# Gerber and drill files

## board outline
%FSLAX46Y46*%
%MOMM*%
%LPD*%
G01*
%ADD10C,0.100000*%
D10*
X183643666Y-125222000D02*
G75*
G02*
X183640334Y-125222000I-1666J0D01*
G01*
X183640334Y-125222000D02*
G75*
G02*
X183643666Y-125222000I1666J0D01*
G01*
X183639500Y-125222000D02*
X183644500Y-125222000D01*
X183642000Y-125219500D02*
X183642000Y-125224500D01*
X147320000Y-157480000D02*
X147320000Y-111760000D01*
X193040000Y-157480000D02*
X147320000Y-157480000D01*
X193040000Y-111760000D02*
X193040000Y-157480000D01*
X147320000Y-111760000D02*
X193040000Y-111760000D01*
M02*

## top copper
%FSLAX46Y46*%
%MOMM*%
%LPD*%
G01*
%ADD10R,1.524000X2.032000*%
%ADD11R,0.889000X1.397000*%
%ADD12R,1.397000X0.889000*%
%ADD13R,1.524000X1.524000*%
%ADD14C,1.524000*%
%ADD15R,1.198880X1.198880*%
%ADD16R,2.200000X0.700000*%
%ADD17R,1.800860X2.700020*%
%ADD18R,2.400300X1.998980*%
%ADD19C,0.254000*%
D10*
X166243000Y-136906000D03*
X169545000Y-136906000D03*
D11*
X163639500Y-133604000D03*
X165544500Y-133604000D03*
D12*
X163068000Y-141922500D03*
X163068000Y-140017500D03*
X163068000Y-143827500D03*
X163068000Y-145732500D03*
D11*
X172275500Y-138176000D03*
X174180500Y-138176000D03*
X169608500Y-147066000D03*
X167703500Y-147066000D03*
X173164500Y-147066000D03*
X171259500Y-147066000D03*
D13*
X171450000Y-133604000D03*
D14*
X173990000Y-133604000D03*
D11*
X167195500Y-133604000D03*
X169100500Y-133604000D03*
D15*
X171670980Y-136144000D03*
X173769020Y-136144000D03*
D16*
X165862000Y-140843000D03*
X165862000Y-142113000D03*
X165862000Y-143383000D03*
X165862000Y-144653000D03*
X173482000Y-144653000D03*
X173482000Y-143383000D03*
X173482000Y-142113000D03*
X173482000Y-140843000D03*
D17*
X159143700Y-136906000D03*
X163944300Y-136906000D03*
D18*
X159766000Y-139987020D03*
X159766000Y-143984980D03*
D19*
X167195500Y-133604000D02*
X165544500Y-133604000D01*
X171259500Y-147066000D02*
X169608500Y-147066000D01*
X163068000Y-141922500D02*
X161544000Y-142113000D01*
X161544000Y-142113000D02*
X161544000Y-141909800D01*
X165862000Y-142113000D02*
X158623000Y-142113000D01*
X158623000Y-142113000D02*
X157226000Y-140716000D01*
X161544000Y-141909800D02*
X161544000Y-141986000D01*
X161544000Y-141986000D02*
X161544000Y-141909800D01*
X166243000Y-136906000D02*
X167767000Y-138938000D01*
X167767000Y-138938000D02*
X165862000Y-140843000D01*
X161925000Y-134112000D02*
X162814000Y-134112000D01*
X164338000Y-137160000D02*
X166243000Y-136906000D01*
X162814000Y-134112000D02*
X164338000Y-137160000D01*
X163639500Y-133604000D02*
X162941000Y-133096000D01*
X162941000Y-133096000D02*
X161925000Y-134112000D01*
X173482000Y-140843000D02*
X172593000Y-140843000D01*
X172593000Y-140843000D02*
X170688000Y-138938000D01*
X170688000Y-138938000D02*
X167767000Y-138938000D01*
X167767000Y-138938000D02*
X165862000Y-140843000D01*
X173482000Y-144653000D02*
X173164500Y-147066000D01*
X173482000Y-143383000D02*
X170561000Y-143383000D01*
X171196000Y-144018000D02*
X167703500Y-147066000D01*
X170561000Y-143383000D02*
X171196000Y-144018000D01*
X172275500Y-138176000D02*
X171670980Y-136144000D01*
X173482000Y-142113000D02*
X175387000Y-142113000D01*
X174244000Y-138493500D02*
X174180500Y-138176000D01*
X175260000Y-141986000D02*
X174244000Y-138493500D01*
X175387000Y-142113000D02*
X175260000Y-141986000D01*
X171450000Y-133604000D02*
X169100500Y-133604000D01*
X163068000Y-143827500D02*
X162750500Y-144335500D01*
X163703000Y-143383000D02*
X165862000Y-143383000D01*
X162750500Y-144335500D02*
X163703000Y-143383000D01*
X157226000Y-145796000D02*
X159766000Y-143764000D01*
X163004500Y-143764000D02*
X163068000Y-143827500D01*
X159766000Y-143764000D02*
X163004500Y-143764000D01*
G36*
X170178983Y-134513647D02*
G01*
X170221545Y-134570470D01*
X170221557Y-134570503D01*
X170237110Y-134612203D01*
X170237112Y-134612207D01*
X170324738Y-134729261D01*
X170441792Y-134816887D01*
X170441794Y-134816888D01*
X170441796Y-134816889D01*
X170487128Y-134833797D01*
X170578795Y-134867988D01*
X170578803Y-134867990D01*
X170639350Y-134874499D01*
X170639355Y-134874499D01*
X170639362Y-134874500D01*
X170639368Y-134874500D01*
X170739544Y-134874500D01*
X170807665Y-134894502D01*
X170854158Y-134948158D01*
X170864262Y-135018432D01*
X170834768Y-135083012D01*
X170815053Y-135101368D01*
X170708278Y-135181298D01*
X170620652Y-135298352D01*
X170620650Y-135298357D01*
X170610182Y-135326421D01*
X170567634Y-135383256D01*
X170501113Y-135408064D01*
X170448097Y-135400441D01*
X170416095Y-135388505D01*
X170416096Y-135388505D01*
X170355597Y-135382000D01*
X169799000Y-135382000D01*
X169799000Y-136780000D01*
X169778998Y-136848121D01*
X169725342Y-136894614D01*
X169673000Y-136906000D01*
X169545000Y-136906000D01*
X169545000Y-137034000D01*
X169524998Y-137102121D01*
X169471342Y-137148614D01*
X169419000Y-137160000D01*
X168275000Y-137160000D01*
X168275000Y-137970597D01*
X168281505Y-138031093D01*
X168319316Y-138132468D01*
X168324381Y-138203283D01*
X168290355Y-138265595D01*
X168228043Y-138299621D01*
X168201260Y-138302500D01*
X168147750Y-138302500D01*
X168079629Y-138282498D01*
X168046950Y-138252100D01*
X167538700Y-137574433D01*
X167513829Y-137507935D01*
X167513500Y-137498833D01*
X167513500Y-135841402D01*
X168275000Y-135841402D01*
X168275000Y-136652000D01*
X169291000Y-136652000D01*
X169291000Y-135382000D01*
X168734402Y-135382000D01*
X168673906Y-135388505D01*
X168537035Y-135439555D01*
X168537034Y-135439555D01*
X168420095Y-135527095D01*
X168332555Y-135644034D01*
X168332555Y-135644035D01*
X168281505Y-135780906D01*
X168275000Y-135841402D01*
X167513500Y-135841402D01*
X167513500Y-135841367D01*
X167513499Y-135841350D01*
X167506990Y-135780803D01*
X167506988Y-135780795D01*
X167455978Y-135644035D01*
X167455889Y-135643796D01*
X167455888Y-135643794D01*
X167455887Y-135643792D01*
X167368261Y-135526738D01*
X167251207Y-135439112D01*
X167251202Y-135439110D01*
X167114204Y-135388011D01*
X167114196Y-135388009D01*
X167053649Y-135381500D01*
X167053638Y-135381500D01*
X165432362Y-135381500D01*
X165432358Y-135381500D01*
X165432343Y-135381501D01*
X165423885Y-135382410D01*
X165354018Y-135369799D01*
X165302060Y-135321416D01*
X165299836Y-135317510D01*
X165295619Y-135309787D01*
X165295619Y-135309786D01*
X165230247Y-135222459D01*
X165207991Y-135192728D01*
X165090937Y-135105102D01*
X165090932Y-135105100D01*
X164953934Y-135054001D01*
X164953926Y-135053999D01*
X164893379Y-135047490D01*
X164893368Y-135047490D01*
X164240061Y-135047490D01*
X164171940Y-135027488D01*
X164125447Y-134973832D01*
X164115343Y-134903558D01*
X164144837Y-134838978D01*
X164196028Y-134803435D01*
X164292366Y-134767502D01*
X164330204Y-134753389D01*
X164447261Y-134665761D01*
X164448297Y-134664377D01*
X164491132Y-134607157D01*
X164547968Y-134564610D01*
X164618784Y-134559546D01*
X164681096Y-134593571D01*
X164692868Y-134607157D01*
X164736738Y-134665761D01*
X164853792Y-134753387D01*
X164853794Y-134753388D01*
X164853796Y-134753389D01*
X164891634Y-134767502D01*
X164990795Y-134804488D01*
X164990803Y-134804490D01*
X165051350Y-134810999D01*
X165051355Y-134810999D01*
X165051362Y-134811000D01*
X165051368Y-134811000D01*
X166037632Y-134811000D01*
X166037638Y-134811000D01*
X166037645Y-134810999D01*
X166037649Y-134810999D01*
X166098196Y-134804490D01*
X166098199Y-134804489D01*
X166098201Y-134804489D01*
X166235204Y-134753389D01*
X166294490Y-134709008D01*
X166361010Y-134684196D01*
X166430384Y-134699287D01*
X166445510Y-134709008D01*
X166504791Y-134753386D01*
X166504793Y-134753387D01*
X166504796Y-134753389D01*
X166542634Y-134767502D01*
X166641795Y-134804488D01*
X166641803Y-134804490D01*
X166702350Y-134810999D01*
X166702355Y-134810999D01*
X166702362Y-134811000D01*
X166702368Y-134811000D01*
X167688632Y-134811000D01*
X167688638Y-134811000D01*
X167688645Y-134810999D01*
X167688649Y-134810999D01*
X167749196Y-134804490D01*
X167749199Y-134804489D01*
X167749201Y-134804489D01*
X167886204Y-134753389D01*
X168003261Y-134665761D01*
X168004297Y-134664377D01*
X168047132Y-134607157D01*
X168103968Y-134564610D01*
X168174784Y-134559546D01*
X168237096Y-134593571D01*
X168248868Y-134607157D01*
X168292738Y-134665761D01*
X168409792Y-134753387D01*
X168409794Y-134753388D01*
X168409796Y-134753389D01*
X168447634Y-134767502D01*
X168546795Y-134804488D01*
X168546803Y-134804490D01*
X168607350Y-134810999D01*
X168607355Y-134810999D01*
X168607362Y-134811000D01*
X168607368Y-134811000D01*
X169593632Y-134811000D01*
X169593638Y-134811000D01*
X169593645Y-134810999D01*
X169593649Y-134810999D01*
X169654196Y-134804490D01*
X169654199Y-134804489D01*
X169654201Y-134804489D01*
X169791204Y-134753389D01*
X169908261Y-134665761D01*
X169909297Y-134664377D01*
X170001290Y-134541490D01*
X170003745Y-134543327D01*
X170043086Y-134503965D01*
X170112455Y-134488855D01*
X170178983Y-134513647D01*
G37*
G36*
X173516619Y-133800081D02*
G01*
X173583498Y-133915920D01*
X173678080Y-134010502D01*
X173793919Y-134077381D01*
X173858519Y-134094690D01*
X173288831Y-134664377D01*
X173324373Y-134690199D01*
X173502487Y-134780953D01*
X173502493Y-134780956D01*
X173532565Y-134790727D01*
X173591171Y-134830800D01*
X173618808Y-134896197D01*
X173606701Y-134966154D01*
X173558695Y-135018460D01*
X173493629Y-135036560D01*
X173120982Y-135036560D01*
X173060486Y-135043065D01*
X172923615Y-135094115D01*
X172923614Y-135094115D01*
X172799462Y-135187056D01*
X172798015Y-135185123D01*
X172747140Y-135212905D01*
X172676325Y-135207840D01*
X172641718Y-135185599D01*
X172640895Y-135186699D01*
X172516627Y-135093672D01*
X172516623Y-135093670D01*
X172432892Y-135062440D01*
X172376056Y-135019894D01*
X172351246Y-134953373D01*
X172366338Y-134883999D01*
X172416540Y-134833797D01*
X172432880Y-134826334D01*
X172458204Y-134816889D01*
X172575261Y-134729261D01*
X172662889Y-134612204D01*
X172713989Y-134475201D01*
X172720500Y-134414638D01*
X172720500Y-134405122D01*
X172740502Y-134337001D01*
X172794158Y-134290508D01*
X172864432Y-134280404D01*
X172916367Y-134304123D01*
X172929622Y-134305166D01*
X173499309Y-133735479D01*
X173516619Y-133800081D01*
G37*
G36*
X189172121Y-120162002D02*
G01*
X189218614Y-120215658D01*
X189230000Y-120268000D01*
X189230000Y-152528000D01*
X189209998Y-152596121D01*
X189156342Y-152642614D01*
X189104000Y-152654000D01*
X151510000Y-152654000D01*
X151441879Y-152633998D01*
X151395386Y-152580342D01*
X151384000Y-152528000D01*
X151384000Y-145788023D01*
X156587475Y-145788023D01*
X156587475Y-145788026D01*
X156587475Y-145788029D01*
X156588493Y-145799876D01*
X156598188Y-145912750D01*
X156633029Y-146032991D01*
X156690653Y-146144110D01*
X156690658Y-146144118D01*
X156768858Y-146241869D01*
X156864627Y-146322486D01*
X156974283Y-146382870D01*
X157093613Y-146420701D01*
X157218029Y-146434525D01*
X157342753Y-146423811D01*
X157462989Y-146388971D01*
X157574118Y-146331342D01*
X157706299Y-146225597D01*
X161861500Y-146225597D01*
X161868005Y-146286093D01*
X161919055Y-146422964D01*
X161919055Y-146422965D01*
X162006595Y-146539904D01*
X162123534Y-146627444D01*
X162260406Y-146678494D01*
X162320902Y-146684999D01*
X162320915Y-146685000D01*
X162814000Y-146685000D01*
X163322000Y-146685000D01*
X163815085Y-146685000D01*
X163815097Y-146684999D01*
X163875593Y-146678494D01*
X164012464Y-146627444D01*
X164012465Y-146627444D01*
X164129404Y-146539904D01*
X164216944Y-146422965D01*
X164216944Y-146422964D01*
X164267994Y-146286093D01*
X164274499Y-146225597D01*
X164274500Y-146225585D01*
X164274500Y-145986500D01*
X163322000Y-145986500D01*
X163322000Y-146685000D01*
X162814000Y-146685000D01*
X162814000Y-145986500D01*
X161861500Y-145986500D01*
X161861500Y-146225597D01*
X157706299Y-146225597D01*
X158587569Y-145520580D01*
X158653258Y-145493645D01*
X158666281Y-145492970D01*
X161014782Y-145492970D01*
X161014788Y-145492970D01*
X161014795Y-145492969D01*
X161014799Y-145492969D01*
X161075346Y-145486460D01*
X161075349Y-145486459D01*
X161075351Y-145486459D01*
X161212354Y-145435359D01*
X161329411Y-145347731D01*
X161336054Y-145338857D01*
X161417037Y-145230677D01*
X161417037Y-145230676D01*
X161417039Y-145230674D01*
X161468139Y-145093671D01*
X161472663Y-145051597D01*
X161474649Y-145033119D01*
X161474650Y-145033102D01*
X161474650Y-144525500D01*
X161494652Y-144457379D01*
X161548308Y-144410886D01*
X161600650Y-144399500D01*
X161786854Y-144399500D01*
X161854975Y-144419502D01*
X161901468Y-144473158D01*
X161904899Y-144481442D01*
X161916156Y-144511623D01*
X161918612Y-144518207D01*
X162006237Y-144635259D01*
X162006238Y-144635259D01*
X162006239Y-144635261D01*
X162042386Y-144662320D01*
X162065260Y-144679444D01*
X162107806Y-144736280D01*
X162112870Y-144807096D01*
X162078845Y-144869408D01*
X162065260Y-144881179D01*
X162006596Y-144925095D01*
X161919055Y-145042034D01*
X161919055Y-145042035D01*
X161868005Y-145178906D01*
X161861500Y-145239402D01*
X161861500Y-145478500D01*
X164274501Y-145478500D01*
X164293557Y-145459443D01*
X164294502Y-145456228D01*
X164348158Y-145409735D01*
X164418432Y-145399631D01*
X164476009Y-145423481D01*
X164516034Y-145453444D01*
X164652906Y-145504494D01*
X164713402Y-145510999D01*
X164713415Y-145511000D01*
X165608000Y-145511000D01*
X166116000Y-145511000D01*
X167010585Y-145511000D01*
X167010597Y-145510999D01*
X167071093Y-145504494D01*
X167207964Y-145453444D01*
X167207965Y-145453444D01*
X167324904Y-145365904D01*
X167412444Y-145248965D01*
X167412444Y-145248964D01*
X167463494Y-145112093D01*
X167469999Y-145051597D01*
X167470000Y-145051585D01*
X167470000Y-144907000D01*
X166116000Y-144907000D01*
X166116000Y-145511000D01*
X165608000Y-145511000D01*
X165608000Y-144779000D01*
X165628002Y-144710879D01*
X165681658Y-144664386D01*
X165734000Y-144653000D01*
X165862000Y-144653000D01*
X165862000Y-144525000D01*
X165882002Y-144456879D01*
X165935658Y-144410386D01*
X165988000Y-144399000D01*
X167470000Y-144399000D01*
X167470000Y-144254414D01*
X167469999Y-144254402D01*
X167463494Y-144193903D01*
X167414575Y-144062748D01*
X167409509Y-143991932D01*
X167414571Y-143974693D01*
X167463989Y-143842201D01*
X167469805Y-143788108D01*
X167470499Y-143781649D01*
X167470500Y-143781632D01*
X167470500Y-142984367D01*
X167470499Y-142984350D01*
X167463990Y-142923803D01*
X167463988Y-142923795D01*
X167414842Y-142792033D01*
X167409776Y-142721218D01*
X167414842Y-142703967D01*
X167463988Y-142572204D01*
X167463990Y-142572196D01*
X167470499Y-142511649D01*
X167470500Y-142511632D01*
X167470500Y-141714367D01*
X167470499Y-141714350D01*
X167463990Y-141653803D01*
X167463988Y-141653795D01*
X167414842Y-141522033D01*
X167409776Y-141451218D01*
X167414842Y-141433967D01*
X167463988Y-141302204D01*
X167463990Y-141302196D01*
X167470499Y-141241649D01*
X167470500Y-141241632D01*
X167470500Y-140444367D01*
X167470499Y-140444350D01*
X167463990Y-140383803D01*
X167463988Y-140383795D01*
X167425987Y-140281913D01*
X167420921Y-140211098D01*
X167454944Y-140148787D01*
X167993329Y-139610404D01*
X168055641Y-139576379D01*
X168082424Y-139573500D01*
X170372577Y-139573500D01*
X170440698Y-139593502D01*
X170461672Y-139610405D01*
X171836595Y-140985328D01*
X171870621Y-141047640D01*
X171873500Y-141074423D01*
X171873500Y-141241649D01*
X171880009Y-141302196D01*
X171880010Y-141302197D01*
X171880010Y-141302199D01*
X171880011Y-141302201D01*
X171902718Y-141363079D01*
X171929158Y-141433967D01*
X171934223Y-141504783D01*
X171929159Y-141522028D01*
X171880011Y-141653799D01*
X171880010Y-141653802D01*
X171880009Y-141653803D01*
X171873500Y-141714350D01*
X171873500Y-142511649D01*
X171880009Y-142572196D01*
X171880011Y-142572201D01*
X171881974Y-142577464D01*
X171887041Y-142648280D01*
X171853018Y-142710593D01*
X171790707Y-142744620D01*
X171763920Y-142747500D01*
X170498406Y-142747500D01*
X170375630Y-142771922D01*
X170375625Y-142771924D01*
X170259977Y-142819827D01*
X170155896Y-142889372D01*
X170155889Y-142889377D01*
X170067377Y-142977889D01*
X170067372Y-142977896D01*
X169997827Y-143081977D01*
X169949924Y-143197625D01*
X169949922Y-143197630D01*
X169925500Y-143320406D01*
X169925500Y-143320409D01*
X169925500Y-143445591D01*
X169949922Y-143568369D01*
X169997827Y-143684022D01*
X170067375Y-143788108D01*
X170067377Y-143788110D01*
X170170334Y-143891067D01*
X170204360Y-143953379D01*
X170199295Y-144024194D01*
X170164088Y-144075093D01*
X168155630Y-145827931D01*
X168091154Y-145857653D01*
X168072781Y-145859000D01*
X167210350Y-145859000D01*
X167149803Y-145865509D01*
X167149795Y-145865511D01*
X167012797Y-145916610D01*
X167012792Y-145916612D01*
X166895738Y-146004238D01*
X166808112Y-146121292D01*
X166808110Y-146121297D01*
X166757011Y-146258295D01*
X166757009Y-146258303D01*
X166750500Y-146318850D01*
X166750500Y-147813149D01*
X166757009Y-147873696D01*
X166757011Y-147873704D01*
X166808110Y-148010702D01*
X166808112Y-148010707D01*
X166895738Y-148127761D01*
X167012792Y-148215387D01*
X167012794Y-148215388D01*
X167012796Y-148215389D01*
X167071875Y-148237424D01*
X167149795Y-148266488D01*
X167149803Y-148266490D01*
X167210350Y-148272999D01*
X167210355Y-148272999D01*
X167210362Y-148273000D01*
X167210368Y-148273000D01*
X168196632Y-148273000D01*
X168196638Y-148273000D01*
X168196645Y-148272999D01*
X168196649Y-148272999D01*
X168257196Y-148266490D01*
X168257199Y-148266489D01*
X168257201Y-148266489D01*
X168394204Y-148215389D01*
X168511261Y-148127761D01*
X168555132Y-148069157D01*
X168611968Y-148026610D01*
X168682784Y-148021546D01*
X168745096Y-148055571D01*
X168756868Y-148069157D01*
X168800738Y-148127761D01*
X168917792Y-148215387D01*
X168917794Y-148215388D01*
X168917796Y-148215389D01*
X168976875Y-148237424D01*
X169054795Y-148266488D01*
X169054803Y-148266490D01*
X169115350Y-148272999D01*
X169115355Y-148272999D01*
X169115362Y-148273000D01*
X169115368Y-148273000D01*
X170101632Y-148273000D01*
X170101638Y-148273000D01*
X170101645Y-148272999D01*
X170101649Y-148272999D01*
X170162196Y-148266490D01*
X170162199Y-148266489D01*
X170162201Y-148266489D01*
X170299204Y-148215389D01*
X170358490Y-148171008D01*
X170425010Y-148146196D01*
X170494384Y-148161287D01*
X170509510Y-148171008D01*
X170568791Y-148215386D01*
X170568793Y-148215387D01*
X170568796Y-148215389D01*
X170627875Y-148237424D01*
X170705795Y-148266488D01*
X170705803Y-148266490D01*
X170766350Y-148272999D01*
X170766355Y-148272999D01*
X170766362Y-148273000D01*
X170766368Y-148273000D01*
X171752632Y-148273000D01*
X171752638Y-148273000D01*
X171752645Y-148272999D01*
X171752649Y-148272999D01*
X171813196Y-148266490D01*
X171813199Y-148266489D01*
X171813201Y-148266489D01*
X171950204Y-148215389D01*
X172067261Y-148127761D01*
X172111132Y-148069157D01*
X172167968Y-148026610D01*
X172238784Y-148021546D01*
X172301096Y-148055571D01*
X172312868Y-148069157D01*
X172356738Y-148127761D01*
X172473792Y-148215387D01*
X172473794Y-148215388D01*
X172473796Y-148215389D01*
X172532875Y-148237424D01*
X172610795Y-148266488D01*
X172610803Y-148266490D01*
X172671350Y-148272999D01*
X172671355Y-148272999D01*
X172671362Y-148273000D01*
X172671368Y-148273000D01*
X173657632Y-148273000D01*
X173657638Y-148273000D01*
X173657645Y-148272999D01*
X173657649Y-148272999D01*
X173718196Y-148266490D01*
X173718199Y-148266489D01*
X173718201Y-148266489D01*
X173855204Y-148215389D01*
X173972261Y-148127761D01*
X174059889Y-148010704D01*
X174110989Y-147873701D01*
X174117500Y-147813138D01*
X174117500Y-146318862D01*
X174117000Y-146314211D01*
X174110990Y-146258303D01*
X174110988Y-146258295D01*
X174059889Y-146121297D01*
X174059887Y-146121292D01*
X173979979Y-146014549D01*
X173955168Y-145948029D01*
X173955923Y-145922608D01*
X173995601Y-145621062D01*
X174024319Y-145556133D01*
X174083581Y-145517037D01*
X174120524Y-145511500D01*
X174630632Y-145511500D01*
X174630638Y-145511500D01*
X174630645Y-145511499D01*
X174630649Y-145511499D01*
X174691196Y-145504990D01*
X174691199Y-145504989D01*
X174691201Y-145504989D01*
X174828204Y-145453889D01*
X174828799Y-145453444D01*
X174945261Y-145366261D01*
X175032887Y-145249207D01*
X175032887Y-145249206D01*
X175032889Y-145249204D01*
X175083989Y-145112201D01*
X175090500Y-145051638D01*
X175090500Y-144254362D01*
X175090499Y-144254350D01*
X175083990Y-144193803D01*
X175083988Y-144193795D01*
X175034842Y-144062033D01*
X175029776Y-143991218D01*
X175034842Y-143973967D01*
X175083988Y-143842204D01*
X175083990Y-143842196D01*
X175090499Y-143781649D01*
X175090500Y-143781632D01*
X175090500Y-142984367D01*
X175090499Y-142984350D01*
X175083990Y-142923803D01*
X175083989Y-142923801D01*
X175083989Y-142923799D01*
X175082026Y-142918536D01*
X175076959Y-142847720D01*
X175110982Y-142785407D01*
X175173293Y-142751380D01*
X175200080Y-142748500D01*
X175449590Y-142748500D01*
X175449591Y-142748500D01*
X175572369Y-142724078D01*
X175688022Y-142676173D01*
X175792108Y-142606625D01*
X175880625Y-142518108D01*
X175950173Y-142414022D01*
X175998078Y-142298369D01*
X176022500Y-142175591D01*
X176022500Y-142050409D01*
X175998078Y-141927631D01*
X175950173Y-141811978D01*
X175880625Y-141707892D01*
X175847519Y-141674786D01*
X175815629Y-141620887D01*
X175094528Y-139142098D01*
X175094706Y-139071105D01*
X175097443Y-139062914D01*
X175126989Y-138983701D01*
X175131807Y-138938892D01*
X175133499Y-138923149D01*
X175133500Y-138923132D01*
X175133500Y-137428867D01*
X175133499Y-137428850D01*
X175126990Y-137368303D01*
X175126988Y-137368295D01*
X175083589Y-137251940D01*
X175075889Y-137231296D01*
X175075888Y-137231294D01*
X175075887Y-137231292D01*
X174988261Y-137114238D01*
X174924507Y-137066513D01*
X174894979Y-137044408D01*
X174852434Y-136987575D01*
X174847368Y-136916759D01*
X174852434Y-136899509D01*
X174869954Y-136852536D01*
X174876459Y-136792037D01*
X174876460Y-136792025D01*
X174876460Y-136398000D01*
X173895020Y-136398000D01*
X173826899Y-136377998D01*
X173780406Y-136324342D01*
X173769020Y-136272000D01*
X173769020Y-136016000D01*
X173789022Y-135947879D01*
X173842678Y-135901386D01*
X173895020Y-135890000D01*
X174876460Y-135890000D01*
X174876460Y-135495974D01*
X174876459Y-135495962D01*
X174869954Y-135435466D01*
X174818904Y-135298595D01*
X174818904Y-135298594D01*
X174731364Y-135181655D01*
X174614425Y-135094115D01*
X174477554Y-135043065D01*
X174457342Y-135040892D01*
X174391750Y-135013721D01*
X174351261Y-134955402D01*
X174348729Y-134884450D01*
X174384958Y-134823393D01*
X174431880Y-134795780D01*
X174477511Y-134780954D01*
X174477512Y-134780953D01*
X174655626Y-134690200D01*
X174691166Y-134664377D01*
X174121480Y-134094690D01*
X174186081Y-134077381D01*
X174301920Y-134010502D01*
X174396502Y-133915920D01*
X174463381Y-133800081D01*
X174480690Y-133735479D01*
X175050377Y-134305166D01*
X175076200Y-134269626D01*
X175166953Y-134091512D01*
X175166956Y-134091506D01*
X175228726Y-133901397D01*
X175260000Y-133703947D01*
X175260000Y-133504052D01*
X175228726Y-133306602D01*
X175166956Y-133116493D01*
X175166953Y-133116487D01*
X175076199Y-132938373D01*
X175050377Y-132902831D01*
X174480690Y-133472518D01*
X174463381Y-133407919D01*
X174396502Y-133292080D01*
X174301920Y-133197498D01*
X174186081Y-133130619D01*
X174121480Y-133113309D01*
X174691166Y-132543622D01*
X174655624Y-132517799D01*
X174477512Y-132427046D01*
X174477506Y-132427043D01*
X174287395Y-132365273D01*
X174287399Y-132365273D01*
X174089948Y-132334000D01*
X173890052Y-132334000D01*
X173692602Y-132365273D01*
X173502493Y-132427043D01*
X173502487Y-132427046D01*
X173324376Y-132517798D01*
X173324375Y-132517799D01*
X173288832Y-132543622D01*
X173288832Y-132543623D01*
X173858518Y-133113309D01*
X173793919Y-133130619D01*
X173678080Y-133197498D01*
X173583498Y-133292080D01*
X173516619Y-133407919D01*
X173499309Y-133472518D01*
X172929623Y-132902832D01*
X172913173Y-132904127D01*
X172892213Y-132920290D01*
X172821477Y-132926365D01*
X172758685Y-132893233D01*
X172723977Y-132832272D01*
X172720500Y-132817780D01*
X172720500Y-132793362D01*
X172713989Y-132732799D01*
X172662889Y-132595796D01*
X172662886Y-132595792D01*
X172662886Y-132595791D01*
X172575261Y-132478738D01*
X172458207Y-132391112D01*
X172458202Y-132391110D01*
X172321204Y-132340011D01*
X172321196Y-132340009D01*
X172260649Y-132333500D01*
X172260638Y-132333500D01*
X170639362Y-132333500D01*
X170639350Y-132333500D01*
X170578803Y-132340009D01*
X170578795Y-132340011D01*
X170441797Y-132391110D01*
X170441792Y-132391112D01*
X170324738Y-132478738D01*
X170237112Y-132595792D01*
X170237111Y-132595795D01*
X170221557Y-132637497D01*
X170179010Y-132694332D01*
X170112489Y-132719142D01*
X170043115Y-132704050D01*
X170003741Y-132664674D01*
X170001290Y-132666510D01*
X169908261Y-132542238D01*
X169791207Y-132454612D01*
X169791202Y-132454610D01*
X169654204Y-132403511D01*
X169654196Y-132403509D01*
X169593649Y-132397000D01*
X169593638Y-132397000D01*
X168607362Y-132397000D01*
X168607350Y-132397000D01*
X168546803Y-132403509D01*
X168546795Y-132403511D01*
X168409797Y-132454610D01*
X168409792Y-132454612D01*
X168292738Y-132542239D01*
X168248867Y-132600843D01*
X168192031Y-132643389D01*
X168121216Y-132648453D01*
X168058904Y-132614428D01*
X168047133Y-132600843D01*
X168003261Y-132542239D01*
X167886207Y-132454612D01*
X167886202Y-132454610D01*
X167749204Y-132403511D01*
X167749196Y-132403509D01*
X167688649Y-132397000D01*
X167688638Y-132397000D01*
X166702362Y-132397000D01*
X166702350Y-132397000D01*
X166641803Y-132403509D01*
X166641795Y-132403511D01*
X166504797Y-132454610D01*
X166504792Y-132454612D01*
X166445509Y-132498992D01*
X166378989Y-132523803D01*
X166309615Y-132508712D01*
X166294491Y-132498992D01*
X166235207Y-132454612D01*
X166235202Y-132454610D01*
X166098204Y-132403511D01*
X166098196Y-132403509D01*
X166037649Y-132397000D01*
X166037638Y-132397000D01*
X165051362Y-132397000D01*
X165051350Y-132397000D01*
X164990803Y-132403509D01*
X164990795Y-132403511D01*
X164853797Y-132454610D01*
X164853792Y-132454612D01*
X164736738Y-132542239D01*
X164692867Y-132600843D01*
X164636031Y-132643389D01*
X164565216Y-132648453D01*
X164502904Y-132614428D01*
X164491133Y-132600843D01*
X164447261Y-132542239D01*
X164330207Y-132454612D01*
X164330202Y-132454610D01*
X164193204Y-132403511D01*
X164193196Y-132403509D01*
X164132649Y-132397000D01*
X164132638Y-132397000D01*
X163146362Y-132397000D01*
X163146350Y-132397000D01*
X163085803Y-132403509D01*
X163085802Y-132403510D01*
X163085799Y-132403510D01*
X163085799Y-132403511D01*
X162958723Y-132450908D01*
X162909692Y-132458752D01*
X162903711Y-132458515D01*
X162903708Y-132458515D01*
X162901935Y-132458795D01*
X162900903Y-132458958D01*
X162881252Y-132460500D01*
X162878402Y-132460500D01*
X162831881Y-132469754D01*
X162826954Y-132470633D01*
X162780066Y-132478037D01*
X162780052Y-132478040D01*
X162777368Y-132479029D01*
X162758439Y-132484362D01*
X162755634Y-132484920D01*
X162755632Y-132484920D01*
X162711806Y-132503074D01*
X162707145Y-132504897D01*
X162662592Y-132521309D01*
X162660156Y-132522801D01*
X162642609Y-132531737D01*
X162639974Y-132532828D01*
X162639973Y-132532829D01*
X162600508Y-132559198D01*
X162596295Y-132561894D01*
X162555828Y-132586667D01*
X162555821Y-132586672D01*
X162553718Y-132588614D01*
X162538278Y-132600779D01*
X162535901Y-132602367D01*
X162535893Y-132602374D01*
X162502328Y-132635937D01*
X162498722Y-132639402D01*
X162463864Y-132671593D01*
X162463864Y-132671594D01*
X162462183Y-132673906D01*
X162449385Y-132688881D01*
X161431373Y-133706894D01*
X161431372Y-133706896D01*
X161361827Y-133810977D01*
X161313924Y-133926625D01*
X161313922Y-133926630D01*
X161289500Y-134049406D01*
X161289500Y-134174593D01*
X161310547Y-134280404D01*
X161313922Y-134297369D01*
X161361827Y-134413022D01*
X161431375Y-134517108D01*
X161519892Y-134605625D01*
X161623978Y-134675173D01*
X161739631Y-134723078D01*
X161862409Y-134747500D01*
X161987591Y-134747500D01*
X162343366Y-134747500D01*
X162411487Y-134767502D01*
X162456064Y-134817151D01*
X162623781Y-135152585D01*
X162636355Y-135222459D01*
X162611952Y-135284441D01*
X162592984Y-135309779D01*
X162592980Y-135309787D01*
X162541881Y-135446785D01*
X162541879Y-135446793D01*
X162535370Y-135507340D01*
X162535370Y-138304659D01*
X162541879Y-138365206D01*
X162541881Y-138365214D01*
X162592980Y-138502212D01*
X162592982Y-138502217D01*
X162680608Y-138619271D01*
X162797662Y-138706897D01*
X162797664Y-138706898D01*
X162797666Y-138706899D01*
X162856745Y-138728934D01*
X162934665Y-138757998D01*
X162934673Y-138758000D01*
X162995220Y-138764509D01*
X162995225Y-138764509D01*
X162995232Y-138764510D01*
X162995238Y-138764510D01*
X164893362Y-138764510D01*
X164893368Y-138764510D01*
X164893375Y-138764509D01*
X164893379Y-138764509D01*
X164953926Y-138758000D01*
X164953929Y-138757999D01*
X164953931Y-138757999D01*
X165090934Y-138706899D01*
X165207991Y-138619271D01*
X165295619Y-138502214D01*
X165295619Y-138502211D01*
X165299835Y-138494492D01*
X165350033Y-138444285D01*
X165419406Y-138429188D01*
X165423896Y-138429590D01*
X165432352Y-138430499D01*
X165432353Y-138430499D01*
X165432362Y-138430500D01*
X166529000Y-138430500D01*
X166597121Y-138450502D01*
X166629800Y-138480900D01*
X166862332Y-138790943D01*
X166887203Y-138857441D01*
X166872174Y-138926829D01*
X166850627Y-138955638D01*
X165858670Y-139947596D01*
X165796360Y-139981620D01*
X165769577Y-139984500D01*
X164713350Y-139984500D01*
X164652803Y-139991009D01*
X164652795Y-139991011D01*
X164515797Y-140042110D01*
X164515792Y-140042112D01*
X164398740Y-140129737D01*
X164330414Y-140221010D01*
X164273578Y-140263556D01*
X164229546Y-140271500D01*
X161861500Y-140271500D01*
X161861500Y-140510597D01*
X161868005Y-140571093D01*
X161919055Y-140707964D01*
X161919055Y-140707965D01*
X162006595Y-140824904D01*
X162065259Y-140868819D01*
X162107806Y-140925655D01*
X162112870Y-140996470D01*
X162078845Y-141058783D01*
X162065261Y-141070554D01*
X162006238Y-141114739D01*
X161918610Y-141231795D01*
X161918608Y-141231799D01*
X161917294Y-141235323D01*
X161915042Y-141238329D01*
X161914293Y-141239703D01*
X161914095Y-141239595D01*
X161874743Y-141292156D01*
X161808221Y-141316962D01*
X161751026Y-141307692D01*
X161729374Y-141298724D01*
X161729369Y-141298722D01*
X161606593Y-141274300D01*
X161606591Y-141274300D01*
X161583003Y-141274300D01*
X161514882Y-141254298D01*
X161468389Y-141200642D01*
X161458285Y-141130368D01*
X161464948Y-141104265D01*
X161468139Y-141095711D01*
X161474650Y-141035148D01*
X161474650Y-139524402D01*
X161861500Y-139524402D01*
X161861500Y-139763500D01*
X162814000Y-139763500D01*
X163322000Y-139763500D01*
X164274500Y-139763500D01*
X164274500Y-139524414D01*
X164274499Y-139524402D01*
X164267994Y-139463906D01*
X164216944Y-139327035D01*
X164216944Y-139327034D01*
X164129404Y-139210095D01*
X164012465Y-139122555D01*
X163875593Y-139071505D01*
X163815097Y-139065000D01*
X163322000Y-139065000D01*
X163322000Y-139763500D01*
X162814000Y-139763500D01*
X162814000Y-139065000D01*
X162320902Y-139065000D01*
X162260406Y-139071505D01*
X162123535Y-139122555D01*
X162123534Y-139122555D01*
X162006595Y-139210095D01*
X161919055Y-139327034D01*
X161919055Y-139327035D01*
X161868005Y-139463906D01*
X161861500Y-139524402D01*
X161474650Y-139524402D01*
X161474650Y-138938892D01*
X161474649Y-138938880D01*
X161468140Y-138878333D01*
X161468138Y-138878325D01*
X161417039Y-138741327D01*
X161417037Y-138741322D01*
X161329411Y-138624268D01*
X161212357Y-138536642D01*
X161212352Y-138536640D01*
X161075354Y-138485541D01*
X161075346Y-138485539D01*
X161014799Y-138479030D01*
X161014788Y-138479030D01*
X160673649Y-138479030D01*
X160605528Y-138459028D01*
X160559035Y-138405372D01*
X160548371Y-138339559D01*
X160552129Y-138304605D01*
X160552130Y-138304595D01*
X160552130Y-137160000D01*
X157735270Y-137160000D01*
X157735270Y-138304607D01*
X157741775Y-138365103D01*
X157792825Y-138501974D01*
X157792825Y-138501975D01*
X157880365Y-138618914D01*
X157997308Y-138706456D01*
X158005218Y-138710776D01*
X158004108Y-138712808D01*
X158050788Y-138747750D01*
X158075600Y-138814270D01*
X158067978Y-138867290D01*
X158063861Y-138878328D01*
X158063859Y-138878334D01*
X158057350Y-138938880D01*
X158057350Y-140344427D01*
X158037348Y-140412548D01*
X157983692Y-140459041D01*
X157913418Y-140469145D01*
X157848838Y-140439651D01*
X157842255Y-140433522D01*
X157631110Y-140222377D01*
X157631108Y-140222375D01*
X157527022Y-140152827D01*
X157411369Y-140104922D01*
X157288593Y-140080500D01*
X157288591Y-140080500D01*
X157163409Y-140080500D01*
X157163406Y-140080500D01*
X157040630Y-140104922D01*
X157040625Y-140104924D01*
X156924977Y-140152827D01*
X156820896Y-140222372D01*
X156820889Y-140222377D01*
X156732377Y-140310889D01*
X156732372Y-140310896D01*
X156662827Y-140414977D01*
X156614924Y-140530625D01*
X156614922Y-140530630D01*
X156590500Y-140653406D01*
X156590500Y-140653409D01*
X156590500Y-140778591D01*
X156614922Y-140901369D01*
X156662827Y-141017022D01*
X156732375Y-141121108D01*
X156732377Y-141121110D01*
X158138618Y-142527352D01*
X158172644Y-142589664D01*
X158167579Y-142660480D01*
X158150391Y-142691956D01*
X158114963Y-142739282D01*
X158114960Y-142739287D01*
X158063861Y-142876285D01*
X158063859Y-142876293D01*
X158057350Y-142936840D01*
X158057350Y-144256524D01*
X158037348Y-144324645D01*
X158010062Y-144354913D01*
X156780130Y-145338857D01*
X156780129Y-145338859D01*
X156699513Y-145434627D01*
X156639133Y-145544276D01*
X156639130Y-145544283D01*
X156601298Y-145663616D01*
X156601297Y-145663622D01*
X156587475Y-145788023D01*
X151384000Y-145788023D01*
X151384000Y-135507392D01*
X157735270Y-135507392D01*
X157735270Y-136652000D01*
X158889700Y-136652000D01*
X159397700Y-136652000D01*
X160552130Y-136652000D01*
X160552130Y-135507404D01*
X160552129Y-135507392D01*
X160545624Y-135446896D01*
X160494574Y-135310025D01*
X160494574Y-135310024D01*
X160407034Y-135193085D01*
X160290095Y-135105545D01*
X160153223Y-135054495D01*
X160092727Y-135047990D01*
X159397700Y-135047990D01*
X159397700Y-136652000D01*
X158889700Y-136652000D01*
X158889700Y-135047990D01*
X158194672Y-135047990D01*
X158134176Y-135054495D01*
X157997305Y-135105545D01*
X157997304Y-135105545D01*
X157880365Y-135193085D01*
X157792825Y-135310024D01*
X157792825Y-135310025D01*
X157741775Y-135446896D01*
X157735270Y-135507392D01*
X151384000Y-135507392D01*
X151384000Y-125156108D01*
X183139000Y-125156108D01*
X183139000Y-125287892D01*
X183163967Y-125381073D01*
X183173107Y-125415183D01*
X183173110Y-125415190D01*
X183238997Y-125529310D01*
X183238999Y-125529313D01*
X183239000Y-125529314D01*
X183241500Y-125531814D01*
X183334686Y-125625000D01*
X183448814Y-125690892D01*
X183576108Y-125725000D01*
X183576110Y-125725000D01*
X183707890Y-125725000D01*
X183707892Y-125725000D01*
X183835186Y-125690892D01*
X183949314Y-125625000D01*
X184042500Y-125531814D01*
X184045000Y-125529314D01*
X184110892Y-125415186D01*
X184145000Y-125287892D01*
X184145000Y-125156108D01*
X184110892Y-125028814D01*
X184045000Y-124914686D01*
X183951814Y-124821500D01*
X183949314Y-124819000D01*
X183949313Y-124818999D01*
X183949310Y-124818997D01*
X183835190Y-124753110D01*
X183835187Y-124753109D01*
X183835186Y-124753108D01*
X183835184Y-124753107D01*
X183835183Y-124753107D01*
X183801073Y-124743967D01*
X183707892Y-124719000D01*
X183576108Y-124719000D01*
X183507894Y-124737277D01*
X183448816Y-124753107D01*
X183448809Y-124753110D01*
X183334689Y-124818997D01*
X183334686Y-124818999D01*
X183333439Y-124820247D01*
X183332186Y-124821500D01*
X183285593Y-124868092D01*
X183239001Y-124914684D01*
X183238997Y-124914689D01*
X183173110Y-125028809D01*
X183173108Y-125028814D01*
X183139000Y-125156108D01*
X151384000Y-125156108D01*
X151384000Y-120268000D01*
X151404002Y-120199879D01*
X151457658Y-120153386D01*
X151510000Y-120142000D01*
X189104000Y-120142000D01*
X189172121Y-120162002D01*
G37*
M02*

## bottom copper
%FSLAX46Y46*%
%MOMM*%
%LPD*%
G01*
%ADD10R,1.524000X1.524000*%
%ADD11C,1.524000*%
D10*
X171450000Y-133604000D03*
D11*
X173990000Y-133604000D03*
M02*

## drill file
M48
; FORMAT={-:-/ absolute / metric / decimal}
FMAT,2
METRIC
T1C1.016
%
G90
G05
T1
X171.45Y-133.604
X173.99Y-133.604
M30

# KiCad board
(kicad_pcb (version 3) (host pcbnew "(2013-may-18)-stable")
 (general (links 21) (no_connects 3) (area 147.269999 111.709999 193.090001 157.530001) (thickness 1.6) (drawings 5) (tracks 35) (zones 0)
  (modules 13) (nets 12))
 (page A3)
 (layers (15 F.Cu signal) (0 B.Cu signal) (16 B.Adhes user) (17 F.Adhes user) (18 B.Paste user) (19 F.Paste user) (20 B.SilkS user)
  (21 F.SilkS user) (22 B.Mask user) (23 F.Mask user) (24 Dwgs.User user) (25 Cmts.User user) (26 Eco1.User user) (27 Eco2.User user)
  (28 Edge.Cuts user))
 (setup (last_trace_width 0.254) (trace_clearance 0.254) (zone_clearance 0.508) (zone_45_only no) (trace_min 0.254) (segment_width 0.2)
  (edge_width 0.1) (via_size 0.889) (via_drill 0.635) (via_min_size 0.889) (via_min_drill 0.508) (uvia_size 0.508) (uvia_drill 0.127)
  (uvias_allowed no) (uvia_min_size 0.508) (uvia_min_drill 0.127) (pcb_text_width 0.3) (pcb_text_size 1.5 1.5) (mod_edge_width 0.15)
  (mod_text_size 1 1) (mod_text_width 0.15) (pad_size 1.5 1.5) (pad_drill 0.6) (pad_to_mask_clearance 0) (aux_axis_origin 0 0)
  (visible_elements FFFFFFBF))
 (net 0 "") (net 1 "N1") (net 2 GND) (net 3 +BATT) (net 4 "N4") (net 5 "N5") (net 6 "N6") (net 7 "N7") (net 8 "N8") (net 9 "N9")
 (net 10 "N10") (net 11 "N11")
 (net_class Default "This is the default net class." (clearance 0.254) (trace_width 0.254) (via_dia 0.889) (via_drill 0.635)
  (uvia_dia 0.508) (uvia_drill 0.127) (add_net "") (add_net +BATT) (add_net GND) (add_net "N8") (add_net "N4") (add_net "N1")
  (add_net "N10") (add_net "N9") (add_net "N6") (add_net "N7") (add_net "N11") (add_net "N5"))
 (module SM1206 (layer F.Cu) (at 167.894 136.906)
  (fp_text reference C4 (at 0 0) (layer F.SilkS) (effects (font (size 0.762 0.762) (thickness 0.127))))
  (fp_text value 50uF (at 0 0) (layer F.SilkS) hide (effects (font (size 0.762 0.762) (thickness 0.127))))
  (pad 1 smd rect (at -1.651 0) (size 1.524 2.032) (layers F.Cu F.Paste F.Mask) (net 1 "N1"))
  (pad 2 smd rect (at 1.651 0) (size 1.524 2.032) (layers F.Cu F.Paste F.Mask) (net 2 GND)))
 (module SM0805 (layer F.Cu) (at 164.592 133.604)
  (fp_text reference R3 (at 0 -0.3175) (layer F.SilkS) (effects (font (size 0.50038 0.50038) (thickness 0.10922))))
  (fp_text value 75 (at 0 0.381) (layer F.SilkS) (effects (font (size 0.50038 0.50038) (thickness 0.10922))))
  (pad 1 smd rect (at -0.9525 0) (size 0.889 1.397) (layers F.Cu F.Paste F.Mask) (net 1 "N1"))
  (pad 2 smd rect (at 0.9525 0) (size 0.889 1.397) (layers F.Cu F.Paste F.Mask) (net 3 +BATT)))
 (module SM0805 (layer F.Cu) (at 163.068 140.97 90)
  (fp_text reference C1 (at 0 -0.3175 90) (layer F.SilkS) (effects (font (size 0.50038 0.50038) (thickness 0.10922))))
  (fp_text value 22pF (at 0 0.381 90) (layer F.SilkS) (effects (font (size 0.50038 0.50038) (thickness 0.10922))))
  (pad 1 smd rect (at -0.9525 0 90) (size 0.889 1.397) (layers F.Cu F.Paste F.Mask) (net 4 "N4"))
  (pad 2 smd rect (at 0.9525 0 90) (size 0.889 1.397) (layers F.Cu F.Paste F.Mask) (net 2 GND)))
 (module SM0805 (layer F.Cu) (at 163.068 144.78 270)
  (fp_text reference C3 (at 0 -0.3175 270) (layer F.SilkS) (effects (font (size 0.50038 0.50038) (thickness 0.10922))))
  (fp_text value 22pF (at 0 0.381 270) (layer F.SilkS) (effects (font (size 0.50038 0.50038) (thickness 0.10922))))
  (pad 1 smd rect (at -0.9525 0 270) (size 0.889 1.397) (layers F.Cu F.Paste F.Mask) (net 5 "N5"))
  (pad 2 smd rect (at 0.9525 0 270) (size 0.889 1.397) (layers F.Cu F.Paste F.Mask) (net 2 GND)))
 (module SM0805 (layer F.Cu) (at 173.228 138.176)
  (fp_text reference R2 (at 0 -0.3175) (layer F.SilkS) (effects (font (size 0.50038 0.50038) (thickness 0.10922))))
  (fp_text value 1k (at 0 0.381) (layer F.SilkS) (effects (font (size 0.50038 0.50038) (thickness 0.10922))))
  (pad 1 smd rect (at -0.9525 0) (size 0.889 1.397) (layers F.Cu F.Paste F.Mask) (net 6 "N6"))
  (pad 2 smd rect (at 0.9525 0) (size 0.889 1.397) (layers F.Cu F.Paste F.Mask) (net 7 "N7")))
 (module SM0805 (layer F.Cu) (at 168.656 147.066 180)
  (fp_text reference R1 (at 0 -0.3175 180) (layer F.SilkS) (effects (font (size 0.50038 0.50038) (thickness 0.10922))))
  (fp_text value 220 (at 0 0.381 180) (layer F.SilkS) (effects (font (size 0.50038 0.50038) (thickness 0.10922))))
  (pad 1 smd rect (at -0.9525 0 180) (size 0.889 1.397) (layers F.Cu F.Paste F.Mask) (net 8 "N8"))
  (pad 2 smd rect (at 0.9525 0 180) (size 0.889 1.397) (layers F.Cu F.Paste F.Mask) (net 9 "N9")))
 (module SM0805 (layer F.Cu) (at 172.212 147.066 180)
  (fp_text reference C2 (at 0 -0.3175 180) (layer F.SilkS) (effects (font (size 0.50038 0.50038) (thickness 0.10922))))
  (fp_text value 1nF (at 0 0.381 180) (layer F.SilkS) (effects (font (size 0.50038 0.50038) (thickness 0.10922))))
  (pad 1 smd rect (at -0.9525 0 180) (size 0.889 1.397) (layers F.Cu F.Paste F.Mask) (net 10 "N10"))
  (pad 2 smd rect (at 0.9525 0 180) (size 0.889 1.397) (layers F.Cu F.Paste F.Mask) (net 8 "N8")))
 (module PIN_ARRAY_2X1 (layer F.Cu) (at 172.72 133.604)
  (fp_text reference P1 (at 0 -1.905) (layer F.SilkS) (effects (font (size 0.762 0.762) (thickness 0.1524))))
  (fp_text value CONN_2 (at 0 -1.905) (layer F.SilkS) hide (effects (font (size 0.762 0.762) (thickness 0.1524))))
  (pad 1 thru_hole rect (at -1.27 0) (size 1.524 1.524) (drill 1.016) (layers *.Cu *.Mask F.SilkS) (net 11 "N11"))
  (pad 2 thru_hole circle (at 1.27 0) (size 1.524 1.524) (drill 1.016) (layers *.Cu *.Mask F.SilkS) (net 2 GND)))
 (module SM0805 (layer F.Cu) (at 168.148 133.604)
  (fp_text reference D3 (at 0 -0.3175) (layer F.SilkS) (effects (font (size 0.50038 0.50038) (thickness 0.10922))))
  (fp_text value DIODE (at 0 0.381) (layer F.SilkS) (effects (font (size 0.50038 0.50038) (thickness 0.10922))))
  (pad 1 smd rect (at -0.9525 0) (size 0.889 1.397) (layers F.Cu F.Paste F.Mask) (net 3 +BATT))
  (pad 2 smd rect (at 0.9525 0) (size 0.889 1.397) (layers F.Cu F.Paste F.Mask) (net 11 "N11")))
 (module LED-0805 (layer F.Cu) (at 172.72 136.144)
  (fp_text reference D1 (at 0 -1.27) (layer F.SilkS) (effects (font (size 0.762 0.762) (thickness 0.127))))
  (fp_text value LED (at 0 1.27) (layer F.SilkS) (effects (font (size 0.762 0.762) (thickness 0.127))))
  (pad 1 smd rect (at -1.04902 0) (size 1.19888 1.19888) (layers F.Cu F.Paste F.Mask) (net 6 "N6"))
  (pad 2 smd rect (at 1.04902 0) (size 1.19888 1.19888) (layers F.Cu F.Paste F.Mask) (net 2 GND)))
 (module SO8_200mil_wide (layer F.Cu) (at 169.672 142.748 270)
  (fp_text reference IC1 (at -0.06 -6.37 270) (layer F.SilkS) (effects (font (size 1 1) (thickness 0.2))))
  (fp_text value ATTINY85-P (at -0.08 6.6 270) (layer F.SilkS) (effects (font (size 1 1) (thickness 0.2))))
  (pad 1 smd rect (at -1.905 3.81 270) (size 0.7 2.2) (layers F.Cu F.Paste F.Mask) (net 1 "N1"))
  (pad 2 smd rect (at -0.635 3.81 270) (size 0.7 2.2) (layers F.Cu F.Paste F.Mask) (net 4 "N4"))
  (pad 3 smd rect (at 0.635 3.81 270) (size 0.7 2.2) (layers F.Cu F.Paste F.Mask) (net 5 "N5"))
  (pad 4 smd rect (at 1.905 3.81 270) (size 0.7 2.2) (layers F.Cu F.Paste F.Mask) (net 2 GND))
  (pad 5 smd rect (at 1.905 -3.81 270) (size 0.7 2.2) (layers F.Cu F.Paste F.Mask) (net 10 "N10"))
  (pad 6 smd rect (at 0.635 -3.81 270) (size 0.7 2.2) (layers F.Cu F.Paste F.Mask) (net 9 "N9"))
  (pad 7 smd rect (at -0.635 -3.81 270) (size 0.7 2.2) (layers F.Cu F.Paste F.Mask) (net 7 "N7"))
  (pad 8 smd rect (at -1.905 -3.81 270) (size 0.7 2.2) (layers F.Cu F.Paste F.Mask) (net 1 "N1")))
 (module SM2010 (layer F.Cu) (at 161.544 136.906)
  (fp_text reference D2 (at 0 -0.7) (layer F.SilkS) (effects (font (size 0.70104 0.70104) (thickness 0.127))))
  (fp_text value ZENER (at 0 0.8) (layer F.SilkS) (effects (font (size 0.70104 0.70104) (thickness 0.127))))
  (pad 1 smd rect (at -2.4003 0) (size 1.80086 2.70002) (layers F.Cu F.Paste F.Mask) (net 2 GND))
  (pad 2 smd rect (at 2.4003 0) (size 1.80086 2.70002) (layers F.Cu F.Paste F.Mask) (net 1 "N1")))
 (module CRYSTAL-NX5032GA (layer F.Cu) (at 159.766 141.986 270)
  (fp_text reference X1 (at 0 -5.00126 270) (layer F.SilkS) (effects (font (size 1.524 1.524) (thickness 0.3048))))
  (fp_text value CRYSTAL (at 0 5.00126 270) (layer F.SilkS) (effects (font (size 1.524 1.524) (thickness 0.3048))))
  (pad 1 smd rect (at -1.99898 0 270) (size 1.99898 2.4003) (layers F.Cu F.Paste F.Mask) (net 4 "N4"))
  (pad 2 smd rect (at 1.99898 0 270) (size 1.99898 2.4003) (layers F.Cu F.Paste F.Mask) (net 5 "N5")))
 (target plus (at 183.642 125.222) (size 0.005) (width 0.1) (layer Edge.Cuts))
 (gr_line (start 147.32 157.48) (end 147.32 111.76) (angle 90) (layer Edge.Cuts) (width 0.1))
 (gr_line (start 193.04 157.48) (end 147.32 157.48) (angle 90) (layer Edge.Cuts) (width 0.1))
 (gr_line (start 193.04 111.76) (end 193.04 157.48) (angle 90) (layer Edge.Cuts) (width 0.1))
 (gr_line (start 147.32 111.76) (end 193.04 111.76) (angle 90) (layer Edge.Cuts) (width 0.1))
 (segment (start 167.1955 133.604) (end 165.5445 133.604) (width 0.254) (layer F.Cu) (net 3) (status 10))
 (segment (start 171.2595 147.066) (end 169.6085 147.066) (width 0.254) (layer F.Cu) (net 8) (status 10))
 (segment (start 163.068 141.9225) (end 161.544 142.113) (width 0.254) (layer F.Cu) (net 4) (status 10))
 (segment (start 161.544 142.113) (end 161.544 141.9098) (width 0.254) (layer F.Cu) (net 4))
 (segment (start 165.862 142.113) (end 158.623 142.113) (width 0.254) (layer F.Cu) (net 4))
 (segment (start 158.623 142.113) (end 157.226 140.716) (width 0.254) (layer F.Cu) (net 4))
 (segment (start 161.544 141.9098) (end 161.544 141.986) (width 0.254) (layer F.Cu) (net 4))
 (segment (start 161.544 141.986) (end 161.544 141.9098) (width 0.254) (layer F.Cu) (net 4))
 (segment (start 166.243 136.906) (end 167.767 138.938) (width 0.254) (layer F.Cu) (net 1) (status 10))
 (segment (start 167.767 138.938) (end 165.862 140.843) (width 0.254) (layer F.Cu) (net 1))
 (segment (start 161.925 134.112) (end 162.814 134.112) (width 0.254) (layer F.Cu) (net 1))
 (segment (start 164.338 137.16) (end 166.243 136.906) (width 0.254) (layer F.Cu) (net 1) (status 20))
 (segment (start 162.814 134.112) (end 164.338 137.16) (width 0.254) (layer F.Cu) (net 1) (status 20))
 (segment (start 163.6395 133.604) (end 162.941 133.096) (width 0.254) (layer F.Cu) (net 1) (status 10))
 (segment (start 162.941 133.096) (end 161.925 134.112) (width 0.254) (layer F.Cu) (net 1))
 (segment (start 173.482 140.843) (end 172.593 140.843) (width 0.254) (layer F.Cu) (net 1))
 (segment (start 172.593 140.843) (end 170.688 138.938) (width 0.254) (layer F.Cu) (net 1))
 (segment (start 170.688 138.938) (end 167.767 138.938) (width 0.254) (layer F.Cu) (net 1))
 (segment (start 167.767 138.938) (end 165.862 140.843) (width 0.254) (layer F.Cu) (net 1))
 (segment (start 173.482 144.653) (end 173.1645 147.066) (width 0.254) (layer F.Cu) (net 10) (status 20))
 (segment (start 173.482 143.383) (end 170.561 143.383) (width 0.254) (layer F.Cu) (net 9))
 (segment (start 171.196 144.018) (end 167.7035 147.066) (width 0.254) (layer F.Cu) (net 9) (status 20))
 (segment (start 170.561 143.383) (end 171.196 144.018) (width 0.254) (layer F.Cu) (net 9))
 (segment (start 172.2755 138.176) (end 171.67098 136.144) (width 0.254) (layer F.Cu) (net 6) (status 10))
 (segment (start 173.482 142.113) (end 175.387 142.113) (width 0.254) (layer F.Cu) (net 7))
 (segment (start 174.244 138.4935) (end 174.1805 138.176) (width 0.254) (layer F.Cu) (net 7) (status 30))
 (segment (start 175.26 141.986) (end 174.244 138.4935) (width 0.254) (layer F.Cu) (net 7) (status 20))
 (segment (start 175.387 142.113) (end 175.26 141.986) (width 0.254) (layer F.Cu) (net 7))
 (segment (start 171.45 133.604) (end 169.1005 133.604) (width 0.254) (layer F.Cu) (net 11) (status 10))
 (segment (start 163.068 143.8275) (end 162.7505 144.3355) (width 0.254) (layer F.Cu) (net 5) (status 10))
 (segment (start 163.703 143.383) (end 165.862 143.383) (width 0.254) (layer F.Cu) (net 5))
 (segment (start 162.7505 144.3355) (end 163.703 143.383) (width 0.254) (layer F.Cu) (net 5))
 (segment (start 157.226 145.796) (end 159.766 143.764) (width 0.254) (layer F.Cu) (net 5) (status 20))
 (segment (start 163.0045 143.764) (end 163.068 143.8275) (width 0.254) (layer F.Cu) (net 5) (status 30))
 (segment (start 159.766 143.764) (end 163.0045 143.764) (width 0.254) (layer F.Cu) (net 5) (status 10))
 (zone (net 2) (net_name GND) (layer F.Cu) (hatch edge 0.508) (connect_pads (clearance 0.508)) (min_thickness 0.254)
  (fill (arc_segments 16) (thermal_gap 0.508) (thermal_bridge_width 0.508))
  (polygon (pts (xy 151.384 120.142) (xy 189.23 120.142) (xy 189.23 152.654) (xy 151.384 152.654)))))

